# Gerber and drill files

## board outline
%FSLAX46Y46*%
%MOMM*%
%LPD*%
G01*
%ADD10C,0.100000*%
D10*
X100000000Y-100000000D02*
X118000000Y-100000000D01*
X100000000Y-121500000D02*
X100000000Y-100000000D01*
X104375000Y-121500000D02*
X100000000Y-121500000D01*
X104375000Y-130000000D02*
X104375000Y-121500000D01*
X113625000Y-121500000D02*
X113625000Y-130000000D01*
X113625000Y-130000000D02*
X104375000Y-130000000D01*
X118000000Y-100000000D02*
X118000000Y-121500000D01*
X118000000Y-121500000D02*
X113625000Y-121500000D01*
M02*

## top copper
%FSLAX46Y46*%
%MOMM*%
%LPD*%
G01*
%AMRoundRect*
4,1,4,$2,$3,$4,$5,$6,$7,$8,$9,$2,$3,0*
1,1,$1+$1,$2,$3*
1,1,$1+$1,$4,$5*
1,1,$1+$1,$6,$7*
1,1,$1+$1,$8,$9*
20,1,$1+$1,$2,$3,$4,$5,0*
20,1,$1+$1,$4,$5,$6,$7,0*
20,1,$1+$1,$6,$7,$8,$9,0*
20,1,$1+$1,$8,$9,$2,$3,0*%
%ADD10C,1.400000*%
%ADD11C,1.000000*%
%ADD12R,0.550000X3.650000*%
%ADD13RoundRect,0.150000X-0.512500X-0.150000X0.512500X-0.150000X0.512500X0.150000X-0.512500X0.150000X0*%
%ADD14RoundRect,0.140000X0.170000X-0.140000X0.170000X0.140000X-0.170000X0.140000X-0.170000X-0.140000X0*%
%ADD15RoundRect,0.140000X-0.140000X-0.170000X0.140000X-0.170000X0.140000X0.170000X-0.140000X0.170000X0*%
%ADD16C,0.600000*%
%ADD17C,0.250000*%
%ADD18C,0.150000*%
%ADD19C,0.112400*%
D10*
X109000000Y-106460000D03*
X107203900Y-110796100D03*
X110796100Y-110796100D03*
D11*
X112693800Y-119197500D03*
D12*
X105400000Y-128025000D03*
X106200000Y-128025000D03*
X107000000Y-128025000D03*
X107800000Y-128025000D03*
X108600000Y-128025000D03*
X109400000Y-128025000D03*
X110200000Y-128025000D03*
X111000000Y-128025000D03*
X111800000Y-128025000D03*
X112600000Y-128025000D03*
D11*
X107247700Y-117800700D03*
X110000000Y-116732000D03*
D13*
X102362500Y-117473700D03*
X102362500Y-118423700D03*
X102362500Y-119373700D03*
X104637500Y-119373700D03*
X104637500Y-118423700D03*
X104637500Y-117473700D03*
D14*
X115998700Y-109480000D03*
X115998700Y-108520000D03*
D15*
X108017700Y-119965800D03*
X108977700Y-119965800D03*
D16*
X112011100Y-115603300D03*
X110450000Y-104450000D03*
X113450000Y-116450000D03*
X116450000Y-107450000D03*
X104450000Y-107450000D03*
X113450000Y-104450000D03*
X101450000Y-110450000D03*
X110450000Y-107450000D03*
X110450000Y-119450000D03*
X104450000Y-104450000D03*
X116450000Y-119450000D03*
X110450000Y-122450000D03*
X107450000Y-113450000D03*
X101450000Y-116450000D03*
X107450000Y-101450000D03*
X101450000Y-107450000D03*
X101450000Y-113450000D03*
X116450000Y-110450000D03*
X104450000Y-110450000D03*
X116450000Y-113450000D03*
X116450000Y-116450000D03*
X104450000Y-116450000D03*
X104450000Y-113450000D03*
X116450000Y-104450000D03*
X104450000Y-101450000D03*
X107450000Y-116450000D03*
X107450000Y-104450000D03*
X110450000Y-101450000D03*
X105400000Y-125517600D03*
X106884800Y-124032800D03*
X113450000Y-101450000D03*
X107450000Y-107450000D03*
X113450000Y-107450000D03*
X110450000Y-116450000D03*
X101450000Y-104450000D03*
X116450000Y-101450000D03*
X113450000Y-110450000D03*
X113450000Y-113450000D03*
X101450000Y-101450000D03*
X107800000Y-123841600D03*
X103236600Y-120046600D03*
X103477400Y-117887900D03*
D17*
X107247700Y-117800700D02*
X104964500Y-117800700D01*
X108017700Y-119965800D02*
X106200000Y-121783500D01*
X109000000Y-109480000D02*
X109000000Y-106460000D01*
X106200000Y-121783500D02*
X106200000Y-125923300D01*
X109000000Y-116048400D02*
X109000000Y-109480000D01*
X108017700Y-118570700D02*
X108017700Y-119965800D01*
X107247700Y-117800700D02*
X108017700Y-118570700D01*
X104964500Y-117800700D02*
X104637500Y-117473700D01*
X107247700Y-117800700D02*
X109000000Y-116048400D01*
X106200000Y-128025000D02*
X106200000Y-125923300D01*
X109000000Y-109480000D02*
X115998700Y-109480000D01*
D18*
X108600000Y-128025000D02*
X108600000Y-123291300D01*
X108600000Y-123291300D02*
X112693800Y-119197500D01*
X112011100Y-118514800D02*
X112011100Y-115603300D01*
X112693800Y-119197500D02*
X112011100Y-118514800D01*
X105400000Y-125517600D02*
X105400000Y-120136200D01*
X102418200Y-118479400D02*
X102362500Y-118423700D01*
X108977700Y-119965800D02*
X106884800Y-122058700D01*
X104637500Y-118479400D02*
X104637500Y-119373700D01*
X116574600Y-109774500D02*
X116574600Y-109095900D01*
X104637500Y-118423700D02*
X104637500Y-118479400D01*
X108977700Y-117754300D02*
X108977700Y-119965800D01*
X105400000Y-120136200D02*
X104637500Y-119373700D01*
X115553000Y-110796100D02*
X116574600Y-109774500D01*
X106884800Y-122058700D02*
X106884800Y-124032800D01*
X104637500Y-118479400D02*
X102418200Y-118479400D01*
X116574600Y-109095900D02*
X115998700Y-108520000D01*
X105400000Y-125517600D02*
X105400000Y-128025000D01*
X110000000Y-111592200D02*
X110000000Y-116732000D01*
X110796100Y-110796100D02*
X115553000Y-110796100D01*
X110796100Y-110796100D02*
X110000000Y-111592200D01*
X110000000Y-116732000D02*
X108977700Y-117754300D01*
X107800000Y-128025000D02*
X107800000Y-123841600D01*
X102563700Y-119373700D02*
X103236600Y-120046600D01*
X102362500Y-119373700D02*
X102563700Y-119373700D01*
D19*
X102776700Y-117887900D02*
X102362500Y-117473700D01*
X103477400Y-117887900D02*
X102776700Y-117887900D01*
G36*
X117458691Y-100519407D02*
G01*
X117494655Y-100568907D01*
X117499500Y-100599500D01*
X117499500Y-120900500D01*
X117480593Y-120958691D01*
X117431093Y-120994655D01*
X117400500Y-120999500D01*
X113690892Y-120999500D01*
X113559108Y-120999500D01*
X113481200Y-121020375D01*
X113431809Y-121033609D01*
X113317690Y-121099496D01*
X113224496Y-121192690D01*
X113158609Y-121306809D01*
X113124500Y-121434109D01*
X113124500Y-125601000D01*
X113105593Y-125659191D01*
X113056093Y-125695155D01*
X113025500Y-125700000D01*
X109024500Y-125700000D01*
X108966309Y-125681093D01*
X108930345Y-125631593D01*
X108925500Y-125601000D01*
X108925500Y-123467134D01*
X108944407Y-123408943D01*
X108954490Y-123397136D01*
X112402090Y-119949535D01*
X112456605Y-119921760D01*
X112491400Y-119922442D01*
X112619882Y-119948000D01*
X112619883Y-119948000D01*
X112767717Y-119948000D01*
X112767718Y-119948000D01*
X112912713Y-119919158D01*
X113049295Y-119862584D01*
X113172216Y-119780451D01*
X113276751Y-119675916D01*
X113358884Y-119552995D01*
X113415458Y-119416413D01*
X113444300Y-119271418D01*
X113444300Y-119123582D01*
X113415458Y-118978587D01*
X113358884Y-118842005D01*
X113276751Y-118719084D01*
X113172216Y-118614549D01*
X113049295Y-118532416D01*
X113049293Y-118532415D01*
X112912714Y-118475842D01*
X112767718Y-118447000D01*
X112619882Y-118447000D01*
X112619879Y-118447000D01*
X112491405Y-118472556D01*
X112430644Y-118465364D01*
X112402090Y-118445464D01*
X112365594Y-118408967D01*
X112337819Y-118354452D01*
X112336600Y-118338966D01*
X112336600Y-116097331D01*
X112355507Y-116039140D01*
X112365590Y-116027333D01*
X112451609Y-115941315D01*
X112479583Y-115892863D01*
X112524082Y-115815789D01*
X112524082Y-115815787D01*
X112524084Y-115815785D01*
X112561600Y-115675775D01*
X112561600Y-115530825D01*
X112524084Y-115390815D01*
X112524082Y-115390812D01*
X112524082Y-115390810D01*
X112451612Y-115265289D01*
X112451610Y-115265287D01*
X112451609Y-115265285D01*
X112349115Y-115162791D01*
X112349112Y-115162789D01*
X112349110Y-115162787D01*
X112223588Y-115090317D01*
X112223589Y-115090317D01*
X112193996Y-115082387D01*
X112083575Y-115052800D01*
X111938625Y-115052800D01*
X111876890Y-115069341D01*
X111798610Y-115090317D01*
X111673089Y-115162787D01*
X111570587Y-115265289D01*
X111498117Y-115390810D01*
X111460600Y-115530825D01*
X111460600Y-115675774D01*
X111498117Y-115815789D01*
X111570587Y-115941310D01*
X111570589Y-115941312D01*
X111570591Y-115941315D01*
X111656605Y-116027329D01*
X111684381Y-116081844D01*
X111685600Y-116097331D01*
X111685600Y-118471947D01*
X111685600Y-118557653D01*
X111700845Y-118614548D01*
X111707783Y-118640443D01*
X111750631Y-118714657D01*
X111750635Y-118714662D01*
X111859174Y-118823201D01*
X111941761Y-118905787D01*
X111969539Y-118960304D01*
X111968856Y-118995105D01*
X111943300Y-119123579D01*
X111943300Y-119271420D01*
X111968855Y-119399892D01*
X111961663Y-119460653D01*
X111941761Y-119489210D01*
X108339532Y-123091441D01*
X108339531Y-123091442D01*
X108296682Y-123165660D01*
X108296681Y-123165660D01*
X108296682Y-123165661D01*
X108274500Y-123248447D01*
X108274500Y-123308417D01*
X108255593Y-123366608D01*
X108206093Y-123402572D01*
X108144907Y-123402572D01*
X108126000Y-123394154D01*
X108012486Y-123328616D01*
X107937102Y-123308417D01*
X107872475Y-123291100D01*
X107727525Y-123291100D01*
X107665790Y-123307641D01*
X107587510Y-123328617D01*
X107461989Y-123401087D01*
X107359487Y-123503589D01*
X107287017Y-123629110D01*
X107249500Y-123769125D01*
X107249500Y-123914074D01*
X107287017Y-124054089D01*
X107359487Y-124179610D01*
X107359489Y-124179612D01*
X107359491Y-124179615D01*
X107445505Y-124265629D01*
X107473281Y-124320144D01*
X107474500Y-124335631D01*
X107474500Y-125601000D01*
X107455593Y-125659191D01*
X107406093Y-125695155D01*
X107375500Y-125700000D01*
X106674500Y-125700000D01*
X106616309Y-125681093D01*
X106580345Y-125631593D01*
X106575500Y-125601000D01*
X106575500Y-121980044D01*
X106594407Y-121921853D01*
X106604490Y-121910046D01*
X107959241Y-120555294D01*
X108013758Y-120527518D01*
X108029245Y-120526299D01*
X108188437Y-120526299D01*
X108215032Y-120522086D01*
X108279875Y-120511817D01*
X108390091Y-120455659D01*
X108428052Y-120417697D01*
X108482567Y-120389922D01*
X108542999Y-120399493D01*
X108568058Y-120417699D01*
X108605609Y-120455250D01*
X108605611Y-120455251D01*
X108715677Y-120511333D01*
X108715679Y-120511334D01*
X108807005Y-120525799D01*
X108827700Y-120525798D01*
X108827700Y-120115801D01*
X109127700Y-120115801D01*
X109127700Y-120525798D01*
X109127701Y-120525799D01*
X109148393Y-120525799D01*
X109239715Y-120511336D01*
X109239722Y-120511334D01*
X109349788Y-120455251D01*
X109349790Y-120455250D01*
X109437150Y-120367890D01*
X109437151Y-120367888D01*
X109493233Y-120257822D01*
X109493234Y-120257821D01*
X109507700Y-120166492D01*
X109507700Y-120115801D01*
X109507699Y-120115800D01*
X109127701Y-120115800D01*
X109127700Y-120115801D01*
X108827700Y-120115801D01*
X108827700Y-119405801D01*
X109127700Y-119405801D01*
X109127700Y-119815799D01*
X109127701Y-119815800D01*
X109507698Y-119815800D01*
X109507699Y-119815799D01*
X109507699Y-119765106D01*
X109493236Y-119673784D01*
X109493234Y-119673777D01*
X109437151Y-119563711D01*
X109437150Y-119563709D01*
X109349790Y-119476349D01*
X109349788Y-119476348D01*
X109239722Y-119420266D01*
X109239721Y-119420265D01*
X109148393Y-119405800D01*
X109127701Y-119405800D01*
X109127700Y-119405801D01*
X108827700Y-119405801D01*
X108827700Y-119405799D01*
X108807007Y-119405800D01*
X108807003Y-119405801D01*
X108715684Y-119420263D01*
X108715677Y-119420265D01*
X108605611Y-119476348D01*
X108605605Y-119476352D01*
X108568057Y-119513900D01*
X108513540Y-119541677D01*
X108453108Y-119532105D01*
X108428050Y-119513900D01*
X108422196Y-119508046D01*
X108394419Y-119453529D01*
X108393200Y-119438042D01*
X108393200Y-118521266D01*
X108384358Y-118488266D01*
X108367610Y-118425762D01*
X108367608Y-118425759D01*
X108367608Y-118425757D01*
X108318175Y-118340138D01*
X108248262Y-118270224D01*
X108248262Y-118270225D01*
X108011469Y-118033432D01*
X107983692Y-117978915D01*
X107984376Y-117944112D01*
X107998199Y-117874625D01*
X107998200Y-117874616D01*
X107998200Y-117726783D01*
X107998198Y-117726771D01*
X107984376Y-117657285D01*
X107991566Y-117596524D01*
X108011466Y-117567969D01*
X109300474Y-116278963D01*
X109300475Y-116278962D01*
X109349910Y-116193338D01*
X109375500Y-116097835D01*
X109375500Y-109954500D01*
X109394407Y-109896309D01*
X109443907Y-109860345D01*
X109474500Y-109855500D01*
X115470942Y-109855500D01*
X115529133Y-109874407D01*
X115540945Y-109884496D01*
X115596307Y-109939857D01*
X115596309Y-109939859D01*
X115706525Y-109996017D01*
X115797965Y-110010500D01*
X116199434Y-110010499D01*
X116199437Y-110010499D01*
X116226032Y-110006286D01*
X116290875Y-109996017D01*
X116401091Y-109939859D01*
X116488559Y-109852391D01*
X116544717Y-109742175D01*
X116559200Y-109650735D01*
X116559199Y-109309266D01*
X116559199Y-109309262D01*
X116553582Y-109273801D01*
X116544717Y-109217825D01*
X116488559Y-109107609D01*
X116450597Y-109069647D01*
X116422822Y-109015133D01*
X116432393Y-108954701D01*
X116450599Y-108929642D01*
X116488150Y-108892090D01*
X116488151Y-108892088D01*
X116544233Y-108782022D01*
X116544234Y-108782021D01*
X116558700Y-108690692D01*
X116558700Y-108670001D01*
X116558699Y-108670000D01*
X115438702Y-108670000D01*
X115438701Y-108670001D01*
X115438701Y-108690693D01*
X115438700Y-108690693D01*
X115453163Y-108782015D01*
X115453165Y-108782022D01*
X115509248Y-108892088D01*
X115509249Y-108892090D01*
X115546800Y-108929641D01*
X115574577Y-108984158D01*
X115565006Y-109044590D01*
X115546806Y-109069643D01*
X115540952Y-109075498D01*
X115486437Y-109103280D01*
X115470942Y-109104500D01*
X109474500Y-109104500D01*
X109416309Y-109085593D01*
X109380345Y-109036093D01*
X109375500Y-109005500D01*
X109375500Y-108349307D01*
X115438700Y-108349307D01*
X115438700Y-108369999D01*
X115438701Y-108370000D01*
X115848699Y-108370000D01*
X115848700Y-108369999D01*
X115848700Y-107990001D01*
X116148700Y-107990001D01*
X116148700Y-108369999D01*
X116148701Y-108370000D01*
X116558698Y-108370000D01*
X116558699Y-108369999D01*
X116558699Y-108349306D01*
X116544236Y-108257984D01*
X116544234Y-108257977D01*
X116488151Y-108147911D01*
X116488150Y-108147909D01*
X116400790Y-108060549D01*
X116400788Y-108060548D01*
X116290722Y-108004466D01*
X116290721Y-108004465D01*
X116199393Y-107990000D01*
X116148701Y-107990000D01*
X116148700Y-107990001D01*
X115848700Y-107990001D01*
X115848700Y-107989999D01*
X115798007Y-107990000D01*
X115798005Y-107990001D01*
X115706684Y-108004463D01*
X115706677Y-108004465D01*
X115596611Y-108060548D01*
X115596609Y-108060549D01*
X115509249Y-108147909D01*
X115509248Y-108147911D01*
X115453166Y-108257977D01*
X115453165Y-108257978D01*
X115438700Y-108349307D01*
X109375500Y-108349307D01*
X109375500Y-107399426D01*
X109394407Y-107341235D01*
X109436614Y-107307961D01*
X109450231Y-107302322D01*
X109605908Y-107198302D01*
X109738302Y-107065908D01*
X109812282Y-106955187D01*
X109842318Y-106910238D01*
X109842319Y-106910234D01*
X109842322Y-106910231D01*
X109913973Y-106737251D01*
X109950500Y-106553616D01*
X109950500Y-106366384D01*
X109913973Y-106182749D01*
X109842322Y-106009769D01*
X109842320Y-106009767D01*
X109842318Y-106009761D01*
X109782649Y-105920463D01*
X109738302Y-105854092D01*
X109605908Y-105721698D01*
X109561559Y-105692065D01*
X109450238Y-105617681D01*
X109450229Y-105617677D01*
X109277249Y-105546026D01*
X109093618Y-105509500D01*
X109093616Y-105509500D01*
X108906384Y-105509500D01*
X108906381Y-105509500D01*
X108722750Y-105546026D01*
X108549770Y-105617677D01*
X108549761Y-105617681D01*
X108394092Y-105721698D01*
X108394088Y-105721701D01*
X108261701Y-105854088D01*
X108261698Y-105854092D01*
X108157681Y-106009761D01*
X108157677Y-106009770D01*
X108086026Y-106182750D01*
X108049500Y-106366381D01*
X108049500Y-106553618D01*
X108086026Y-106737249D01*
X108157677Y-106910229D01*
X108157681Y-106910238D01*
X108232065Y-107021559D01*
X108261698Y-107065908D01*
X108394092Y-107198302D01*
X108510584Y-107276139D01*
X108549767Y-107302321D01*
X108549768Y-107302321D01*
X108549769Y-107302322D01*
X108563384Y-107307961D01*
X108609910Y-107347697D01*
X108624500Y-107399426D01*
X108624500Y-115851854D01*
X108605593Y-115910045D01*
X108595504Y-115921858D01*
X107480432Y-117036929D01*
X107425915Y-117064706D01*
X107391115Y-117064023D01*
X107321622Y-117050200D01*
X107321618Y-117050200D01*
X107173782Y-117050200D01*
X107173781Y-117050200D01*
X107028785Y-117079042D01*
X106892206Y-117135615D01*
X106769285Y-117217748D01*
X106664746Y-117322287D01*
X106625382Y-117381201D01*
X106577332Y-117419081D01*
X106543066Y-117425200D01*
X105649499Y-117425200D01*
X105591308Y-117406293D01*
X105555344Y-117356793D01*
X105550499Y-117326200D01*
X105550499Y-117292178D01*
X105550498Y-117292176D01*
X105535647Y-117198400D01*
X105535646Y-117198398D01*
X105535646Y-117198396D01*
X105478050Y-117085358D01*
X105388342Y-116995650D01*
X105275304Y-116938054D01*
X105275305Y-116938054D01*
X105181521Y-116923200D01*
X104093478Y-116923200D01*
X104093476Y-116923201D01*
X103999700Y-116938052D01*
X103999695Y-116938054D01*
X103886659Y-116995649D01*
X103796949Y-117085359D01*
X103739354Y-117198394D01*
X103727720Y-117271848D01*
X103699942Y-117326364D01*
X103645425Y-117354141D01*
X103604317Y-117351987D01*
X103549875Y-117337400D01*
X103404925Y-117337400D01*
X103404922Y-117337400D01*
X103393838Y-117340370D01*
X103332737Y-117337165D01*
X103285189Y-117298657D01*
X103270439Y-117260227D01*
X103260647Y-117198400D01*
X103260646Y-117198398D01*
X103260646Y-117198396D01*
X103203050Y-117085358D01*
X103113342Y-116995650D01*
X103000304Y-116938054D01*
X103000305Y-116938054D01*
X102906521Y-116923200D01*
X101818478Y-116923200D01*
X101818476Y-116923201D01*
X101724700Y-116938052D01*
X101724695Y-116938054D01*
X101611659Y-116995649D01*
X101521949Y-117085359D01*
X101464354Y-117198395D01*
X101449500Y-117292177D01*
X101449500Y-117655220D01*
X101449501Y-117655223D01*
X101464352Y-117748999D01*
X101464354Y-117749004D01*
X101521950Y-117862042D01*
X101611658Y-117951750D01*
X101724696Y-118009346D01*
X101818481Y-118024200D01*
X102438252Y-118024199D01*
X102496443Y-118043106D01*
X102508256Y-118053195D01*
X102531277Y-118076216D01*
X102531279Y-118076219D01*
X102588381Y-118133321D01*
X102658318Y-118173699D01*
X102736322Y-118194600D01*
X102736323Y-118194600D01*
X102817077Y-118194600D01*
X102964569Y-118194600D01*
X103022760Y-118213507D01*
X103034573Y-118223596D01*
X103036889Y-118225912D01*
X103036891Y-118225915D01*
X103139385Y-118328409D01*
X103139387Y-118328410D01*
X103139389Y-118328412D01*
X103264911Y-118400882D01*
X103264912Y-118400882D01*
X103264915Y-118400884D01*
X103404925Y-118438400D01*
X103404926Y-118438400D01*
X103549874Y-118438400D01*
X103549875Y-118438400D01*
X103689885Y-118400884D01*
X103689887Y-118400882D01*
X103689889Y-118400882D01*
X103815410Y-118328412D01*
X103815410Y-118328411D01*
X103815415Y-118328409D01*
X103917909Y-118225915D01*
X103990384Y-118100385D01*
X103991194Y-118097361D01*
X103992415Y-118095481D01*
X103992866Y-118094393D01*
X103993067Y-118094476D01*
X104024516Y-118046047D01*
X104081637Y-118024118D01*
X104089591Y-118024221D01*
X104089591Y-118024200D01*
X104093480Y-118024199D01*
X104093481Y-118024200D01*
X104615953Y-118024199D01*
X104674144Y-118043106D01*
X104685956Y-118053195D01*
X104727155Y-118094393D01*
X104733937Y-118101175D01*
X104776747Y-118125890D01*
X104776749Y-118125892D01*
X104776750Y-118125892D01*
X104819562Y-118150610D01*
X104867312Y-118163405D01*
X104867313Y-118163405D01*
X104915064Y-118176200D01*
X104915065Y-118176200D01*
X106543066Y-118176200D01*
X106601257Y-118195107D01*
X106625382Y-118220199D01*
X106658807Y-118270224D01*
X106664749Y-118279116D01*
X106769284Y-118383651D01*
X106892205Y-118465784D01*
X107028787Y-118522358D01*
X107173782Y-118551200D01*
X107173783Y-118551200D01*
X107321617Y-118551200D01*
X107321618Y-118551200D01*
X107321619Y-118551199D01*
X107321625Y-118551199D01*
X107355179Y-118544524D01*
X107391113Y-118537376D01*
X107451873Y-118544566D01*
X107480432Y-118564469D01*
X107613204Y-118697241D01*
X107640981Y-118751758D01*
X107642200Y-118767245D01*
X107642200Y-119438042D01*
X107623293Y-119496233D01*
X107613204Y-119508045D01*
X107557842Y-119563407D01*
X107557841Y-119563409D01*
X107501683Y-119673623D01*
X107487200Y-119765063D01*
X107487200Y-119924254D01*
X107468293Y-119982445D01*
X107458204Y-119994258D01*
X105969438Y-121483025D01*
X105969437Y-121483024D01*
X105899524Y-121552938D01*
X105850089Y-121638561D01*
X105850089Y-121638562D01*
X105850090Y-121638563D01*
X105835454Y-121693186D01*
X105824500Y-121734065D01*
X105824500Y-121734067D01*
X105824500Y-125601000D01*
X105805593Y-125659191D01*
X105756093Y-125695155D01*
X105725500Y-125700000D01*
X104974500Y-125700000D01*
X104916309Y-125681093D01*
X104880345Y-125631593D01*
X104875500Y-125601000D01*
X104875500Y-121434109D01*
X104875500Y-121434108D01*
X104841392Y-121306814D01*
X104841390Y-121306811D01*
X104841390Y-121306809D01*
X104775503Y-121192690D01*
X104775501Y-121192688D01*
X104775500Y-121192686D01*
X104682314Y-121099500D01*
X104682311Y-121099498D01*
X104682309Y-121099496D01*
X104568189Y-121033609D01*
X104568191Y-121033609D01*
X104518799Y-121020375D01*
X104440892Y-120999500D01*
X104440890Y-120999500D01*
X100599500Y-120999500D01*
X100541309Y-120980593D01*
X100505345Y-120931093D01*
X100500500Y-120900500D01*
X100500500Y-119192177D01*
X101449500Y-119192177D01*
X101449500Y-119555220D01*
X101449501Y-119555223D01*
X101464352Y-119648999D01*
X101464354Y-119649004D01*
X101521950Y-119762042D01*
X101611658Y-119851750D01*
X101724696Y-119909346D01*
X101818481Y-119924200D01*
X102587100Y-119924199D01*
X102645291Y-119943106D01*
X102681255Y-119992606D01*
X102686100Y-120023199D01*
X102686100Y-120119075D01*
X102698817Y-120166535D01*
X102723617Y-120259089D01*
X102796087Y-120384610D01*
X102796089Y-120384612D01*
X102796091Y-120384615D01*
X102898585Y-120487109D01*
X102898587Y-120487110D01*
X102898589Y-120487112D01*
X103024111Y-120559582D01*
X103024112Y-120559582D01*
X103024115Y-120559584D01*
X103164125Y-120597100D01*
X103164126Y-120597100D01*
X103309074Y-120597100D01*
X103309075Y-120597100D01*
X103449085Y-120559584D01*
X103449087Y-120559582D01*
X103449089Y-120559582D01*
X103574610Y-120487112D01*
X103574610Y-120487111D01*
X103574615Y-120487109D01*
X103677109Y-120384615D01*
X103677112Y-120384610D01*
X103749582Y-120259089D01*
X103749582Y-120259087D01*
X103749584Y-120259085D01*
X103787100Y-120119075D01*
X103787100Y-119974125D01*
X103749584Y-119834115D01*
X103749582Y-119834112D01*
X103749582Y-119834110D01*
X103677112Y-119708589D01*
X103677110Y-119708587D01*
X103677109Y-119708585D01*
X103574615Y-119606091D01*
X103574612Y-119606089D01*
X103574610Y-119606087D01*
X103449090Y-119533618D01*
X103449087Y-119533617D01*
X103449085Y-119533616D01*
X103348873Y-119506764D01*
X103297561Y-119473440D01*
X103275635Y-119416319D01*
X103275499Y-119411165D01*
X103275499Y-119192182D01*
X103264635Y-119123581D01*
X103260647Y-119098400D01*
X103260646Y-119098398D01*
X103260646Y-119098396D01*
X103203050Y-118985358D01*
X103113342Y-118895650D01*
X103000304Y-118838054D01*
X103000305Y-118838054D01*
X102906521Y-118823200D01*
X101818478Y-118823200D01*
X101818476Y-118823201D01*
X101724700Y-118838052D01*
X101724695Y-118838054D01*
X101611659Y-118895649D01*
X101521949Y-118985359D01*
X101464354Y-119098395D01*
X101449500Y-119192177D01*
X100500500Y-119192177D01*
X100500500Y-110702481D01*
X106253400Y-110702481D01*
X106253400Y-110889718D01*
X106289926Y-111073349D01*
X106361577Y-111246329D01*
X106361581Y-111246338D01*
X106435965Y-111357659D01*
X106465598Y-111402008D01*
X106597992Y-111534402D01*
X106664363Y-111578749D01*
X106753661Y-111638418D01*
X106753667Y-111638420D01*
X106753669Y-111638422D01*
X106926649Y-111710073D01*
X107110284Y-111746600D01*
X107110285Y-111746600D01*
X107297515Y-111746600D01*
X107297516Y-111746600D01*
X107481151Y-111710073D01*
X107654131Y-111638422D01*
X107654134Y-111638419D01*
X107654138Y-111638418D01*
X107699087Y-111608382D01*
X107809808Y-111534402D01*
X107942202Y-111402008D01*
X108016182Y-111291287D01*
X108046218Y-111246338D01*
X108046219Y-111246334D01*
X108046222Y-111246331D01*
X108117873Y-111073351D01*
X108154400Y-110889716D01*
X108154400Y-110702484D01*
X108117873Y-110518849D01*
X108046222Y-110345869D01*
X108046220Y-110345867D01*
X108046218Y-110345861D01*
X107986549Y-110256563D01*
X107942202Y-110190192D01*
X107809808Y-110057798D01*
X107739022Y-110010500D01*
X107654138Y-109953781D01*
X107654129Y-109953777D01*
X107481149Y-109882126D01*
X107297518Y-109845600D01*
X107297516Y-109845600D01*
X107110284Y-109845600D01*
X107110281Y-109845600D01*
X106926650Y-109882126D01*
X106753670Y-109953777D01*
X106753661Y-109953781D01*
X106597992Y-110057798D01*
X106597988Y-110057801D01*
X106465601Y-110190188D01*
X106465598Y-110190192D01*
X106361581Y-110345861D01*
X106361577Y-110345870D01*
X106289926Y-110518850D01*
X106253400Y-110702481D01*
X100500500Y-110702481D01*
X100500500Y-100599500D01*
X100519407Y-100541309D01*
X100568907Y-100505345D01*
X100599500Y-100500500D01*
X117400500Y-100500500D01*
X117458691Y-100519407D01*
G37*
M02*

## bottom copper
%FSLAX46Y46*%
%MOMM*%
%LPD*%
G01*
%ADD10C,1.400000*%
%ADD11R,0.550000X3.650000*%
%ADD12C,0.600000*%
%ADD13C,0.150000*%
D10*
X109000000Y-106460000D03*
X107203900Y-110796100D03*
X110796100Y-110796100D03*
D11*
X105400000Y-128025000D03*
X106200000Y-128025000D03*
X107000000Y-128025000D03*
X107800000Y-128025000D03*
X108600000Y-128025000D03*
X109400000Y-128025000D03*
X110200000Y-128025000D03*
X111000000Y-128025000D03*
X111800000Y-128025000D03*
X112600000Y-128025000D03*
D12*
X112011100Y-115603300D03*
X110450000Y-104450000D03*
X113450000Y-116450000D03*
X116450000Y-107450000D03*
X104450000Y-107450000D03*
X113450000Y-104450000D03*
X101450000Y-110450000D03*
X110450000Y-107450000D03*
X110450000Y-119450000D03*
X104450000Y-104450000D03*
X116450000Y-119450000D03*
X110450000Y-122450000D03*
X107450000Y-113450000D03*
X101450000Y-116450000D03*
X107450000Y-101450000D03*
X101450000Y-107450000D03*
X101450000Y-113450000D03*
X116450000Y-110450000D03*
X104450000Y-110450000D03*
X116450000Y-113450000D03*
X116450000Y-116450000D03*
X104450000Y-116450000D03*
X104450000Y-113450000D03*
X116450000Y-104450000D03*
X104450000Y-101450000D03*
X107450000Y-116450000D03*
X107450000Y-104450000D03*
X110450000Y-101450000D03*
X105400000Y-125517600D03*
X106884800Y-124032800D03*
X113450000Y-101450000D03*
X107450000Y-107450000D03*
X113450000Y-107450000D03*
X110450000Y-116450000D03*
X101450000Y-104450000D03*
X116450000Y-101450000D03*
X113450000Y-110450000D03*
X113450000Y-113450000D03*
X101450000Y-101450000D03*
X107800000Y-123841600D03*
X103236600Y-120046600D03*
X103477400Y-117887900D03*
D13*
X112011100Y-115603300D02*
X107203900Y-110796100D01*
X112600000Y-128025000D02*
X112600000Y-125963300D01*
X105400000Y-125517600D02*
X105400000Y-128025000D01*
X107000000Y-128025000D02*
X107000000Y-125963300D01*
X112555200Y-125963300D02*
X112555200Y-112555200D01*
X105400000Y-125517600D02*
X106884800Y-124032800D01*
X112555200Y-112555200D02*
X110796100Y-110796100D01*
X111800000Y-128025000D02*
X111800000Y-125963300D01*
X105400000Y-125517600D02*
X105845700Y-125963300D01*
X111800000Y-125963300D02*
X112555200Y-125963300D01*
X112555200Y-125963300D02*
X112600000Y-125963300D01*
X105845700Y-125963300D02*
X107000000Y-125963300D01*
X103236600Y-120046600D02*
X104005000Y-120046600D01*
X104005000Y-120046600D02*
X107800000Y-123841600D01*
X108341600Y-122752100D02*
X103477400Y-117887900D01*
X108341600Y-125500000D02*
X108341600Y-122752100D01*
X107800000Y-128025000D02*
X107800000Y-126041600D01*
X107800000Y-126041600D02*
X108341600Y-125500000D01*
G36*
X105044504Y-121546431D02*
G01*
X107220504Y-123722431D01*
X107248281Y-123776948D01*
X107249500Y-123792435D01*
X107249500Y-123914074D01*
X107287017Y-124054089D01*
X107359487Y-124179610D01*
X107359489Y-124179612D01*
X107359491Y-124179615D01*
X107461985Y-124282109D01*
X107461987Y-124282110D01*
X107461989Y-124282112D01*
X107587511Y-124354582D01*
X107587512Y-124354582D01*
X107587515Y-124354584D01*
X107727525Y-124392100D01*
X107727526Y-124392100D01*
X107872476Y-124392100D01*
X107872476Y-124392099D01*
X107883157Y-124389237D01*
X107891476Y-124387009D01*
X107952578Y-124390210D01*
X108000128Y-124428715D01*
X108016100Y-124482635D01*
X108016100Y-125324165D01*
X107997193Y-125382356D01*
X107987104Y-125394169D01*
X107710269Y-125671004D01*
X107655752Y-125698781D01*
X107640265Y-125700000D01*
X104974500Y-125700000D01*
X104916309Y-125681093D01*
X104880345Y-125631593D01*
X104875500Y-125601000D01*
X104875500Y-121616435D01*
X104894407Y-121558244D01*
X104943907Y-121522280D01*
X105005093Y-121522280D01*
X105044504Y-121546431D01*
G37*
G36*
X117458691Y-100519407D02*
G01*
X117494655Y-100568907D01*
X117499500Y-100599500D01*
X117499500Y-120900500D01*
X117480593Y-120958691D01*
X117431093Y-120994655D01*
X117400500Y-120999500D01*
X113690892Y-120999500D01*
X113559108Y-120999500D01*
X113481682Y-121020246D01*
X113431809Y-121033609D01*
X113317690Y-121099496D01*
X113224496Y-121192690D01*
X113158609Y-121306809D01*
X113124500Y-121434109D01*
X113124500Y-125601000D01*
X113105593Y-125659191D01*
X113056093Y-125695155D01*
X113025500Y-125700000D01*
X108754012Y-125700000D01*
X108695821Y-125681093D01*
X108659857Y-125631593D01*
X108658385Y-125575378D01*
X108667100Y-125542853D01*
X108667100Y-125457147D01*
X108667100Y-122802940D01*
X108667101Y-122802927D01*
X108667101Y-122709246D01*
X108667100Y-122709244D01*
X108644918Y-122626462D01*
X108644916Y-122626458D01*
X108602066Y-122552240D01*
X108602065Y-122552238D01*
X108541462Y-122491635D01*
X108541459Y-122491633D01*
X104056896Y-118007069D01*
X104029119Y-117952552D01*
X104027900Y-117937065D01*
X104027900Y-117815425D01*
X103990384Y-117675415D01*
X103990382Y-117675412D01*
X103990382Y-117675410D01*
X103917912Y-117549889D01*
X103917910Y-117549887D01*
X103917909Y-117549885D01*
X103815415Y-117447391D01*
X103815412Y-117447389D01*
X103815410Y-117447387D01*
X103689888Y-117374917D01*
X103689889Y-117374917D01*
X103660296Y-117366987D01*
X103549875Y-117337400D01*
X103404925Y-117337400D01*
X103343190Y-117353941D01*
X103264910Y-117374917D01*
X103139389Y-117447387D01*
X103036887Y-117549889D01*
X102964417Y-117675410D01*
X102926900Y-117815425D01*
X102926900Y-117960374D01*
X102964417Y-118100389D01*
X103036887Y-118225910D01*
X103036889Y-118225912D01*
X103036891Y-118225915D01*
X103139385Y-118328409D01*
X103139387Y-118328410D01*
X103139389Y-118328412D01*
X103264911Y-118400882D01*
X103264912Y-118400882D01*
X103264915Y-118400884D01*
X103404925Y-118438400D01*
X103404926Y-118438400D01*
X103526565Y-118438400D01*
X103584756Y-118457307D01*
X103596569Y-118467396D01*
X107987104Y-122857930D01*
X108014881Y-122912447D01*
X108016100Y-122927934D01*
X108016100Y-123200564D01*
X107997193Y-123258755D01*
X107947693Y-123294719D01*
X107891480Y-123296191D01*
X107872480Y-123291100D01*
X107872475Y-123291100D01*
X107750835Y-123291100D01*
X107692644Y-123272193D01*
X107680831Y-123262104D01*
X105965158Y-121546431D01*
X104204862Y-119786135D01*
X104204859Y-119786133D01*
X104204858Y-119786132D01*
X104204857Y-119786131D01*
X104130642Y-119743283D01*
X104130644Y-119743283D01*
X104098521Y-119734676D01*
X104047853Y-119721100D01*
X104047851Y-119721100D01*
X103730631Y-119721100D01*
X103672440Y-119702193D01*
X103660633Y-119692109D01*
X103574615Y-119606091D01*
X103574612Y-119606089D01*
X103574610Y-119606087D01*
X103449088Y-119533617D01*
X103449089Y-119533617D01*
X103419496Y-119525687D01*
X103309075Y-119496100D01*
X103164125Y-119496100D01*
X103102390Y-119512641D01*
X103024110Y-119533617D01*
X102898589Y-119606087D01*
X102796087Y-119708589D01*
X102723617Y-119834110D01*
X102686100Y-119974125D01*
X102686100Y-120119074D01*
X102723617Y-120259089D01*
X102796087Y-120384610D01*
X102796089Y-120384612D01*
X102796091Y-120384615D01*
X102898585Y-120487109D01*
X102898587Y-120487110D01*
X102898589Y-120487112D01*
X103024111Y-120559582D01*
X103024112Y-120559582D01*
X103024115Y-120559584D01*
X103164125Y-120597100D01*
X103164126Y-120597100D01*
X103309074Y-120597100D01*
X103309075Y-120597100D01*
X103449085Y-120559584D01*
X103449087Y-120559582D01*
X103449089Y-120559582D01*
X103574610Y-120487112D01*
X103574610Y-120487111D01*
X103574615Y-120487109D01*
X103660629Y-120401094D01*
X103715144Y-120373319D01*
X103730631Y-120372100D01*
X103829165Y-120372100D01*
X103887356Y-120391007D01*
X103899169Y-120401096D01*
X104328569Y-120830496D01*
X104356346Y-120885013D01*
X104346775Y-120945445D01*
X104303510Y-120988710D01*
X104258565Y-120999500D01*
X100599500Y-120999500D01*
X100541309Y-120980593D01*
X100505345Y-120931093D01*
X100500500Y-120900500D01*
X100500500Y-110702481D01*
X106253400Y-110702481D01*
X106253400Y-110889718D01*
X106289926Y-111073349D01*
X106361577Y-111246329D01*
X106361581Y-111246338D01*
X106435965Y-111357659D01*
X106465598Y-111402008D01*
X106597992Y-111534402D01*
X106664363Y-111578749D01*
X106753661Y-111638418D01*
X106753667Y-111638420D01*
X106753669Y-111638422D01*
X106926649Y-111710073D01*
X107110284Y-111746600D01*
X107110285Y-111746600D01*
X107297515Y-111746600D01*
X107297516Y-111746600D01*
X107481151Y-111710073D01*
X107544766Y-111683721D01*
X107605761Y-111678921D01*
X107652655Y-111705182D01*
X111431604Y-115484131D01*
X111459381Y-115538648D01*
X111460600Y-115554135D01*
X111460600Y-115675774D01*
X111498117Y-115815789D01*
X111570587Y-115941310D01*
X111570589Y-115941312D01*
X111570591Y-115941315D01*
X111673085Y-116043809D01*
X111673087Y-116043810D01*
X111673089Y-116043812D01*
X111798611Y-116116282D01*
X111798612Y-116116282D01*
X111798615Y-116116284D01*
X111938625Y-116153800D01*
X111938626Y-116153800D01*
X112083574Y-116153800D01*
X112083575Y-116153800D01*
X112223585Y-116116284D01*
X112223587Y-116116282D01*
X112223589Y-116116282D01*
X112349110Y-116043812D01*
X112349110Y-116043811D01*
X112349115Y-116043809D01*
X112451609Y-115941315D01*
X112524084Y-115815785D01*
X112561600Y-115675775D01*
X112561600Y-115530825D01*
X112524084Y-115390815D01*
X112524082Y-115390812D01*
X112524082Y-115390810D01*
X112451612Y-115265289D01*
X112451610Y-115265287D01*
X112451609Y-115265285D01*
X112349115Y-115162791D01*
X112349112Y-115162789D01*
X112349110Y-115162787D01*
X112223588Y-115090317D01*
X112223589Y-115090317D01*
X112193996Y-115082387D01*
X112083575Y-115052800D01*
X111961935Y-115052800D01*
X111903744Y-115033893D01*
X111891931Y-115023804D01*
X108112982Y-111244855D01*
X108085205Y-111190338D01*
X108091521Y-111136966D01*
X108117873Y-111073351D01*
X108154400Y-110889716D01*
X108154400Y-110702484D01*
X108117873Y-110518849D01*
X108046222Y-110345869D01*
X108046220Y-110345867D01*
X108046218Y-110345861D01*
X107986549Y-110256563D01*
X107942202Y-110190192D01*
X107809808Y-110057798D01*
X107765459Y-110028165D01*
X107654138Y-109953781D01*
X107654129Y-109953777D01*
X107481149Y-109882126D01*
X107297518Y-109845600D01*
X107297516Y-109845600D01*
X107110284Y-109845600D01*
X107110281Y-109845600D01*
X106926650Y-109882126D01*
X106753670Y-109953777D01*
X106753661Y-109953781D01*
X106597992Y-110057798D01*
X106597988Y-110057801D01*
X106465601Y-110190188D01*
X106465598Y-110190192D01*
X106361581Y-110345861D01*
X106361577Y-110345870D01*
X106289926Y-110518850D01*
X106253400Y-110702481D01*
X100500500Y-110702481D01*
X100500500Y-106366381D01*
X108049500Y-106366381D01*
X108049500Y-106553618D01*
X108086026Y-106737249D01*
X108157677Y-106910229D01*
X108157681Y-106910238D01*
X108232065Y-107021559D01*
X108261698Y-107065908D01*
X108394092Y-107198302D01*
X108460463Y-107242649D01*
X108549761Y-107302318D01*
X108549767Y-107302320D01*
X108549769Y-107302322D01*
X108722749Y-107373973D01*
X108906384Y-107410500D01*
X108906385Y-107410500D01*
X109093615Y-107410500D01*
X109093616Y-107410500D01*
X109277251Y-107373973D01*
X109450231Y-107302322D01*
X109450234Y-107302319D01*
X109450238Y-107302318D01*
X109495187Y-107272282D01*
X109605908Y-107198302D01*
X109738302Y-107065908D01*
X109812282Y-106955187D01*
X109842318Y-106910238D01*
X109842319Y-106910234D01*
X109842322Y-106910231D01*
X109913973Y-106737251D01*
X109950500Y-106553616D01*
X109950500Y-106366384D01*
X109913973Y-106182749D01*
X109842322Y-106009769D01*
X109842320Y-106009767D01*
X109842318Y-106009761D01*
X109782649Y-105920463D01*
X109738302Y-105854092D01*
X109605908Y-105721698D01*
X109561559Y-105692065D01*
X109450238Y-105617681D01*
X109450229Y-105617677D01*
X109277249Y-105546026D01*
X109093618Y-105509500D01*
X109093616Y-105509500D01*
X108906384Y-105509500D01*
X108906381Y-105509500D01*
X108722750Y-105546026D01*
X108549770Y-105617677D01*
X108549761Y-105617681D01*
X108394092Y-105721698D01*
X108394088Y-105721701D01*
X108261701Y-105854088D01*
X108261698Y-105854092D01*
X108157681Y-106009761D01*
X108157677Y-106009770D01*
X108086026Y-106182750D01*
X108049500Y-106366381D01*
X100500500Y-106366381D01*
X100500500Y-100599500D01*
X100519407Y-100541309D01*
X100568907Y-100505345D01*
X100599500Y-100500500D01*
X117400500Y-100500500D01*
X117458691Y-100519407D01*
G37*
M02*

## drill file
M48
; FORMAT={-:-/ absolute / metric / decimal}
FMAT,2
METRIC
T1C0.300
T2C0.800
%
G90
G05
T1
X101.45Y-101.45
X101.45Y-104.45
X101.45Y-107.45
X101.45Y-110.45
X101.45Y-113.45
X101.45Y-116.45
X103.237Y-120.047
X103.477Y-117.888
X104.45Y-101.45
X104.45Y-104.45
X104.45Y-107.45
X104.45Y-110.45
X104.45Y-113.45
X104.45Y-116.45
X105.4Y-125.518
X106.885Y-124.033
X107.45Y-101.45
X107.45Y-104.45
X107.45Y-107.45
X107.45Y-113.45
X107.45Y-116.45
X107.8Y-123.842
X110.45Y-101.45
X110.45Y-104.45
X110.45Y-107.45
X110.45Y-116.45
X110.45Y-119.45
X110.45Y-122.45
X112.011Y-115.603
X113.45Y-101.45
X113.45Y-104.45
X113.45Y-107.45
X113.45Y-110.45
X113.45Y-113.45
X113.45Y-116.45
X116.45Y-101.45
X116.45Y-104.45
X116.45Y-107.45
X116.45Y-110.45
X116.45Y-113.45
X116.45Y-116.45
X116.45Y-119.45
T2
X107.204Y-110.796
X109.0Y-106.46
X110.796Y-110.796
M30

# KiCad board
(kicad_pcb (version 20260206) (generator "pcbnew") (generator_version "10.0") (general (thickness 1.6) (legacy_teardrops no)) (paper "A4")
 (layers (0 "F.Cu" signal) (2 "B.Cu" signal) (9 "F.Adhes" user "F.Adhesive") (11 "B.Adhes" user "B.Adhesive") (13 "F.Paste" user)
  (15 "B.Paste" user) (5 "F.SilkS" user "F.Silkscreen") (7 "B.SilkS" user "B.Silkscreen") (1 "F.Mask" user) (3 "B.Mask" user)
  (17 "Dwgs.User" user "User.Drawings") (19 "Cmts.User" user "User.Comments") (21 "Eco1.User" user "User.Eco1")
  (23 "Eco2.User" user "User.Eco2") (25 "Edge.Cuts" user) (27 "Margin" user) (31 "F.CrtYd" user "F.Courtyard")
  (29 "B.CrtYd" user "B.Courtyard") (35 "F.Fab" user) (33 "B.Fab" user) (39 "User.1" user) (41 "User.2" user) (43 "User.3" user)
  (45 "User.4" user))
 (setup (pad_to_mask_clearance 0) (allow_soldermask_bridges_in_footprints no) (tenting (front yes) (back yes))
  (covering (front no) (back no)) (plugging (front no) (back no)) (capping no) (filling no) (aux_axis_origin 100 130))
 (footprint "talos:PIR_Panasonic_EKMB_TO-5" (layer "F.Cu") (at 109 109)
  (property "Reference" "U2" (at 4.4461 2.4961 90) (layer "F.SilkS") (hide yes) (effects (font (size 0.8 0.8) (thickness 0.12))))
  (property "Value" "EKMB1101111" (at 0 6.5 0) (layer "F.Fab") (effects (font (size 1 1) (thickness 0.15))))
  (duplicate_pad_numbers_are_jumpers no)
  (pad "1" thru_hole circle (at 0 -2.54) (size 1.4 1.4) (drill 0.8) (layers "*.Cu" "*.Mask") (remove_unused_layers no) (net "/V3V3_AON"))
  (pad "2" thru_hole circle (at -1.7961 1.7961) (size 1.4 1.4) (drill 0.8) (layers "*.Cu" "*.Mask") (remove_unused_layers no) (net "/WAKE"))
  (pad "3" thru_hole circle (at 1.7961 1.7961) (size 1.4 1.4) (drill 0.8) (layers "*.Cu" "*.Mask") (remove_unused_layers no) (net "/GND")))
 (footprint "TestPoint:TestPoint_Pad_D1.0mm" (layer "F.Cu") (at 112.6938 119.1975)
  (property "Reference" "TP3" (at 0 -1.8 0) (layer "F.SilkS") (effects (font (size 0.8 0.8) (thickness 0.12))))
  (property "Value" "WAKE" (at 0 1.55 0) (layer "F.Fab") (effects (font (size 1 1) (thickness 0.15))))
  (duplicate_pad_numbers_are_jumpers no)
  (pad "1" smd circle (at 0 0) (size 1 1) (layers "F.Cu" "F.Mask") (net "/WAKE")))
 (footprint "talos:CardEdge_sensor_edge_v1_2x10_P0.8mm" (layer "F.Cu") (at 109 128.35)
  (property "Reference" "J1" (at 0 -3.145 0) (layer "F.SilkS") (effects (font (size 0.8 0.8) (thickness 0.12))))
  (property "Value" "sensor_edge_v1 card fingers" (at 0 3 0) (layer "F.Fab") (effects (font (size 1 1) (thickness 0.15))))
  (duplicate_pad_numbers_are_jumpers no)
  (pad "1" smd rect (at -3.6 -0.325) (size 0.55 3.65) (layers "F.Cu" "F.Mask") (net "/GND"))
  (pad "2" smd rect (at -3.6 -0.325) (size 0.55 3.65) (layers "B.Cu" "B.Mask") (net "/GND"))
  (pad "3" smd rect (at -2.8 -0.325) (size 0.55 3.65) (layers "F.Cu" "F.Mask") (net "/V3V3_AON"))
  (pad "4" smd rect (at -2.8 -0.325) (size 0.55 3.65) (layers "B.Cu" "B.Mask") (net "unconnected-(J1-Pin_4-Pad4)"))
  (pad "5" smd rect (at -2 -0.325) (size 0.55 3.65) (layers "F.Cu" "F.Mask") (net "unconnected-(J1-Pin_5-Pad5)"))
  (pad "6" smd rect (at -2 -0.325) (size 0.55 3.65) (layers "B.Cu" "B.Mask") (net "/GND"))
  (pad "7" smd rect (at -1.2 -0.325) (size 0.55 3.65) (layers "F.Cu" "F.Mask") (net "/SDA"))
  (pad "8" smd rect (at -1.2 -0.325) (size 0.55 3.65) (layers "B.Cu" "B.Mask") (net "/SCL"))
  (pad "9" smd rect (at -0.4 -0.325) (size 0.55 3.65) (layers "F.Cu" "F.Mask") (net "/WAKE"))
  (pad "10" smd rect (at -0.4 -0.325) (size 0.55 3.65) (layers "B.Cu" "B.Mask") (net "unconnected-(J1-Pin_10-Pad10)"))
  (pad "11" smd rect (at 0.4 -0.325) (size 0.55 3.65) (layers "F.Cu" "F.Mask") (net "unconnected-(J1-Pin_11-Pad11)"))
  (pad "12" smd rect (at 0.4 -0.325) (size 0.55 3.65) (layers "B.Cu" "B.Mask") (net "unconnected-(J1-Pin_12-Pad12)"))
  (pad "13" smd rect (at 1.2 -0.325) (size 0.55 3.65) (layers "F.Cu" "F.Mask") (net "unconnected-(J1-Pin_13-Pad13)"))
  (pad "14" smd rect (at 1.2 -0.325) (size 0.55 3.65) (layers "B.Cu" "B.Mask") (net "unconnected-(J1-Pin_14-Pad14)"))
  (pad "15" smd rect (at 2 -0.325) (size 0.55 3.65) (layers "F.Cu" "F.Mask") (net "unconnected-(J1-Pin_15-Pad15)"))
  (pad "16" smd rect (at 2 -0.325) (size 0.55 3.65) (layers "B.Cu" "B.Mask") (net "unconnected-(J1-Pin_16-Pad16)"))
  (pad "17" smd rect (at 2.8 -0.325) (size 0.55 3.65) (layers "F.Cu" "F.Mask") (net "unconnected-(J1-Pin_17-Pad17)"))
  (pad "18" smd rect (at 2.8 -0.325) (size 0.55 3.65) (layers "B.Cu" "B.Mask") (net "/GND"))
  (pad "19" smd rect (at 3.6 -0.325) (size 0.55 3.65) (layers "F.Cu" "F.Mask") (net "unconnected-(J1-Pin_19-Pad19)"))
  (pad "20" smd rect (at 3.6 -0.325) (size 0.55 3.65) (layers "B.Cu" "B.Mask") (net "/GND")))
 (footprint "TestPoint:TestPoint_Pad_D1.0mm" (layer "F.Cu") (at 107.2477 117.8007)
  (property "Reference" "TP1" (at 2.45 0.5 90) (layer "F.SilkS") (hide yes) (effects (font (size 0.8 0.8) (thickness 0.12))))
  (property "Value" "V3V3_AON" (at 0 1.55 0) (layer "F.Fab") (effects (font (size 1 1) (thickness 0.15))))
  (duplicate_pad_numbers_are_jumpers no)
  (pad "1" smd circle (at 0 0) (size 1 1) (layers "F.Cu" "F.Mask") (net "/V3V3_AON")))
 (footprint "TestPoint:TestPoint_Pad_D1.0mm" (layer "F.Cu") (at 110 116.732)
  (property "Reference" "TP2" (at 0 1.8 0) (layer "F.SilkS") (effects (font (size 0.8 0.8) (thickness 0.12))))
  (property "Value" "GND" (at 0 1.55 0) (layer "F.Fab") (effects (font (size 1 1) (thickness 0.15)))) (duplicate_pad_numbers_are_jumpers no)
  (pad "1" smd circle (at 0 0) (size 1 1) (layers "F.Cu" "F.Mask") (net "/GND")))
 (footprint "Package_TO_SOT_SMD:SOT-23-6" (layer "F.Cu") (at 103.5 118.4237)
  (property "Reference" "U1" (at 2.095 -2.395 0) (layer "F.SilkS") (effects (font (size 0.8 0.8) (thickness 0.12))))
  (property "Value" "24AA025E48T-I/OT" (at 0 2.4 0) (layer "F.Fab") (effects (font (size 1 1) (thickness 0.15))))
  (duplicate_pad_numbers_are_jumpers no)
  (pad "1" smd roundrect (at -1.1375 -0.95) (size 1.325 0.6) (layers "F.Cu" "F.Mask" "F.Paste") (roundrect_rratio 0.25) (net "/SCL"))
  (pad "2" smd roundrect (at -1.1375 0) (size 1.325 0.6) (layers "F.Cu" "F.Mask" "F.Paste") (roundrect_rratio 0.25) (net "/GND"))
  (pad "3" smd roundrect (at -1.1375 0.95) (size 1.325 0.6) (layers "F.Cu" "F.Mask" "F.Paste") (roundrect_rratio 0.25) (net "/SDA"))
  (pad "4" smd roundrect (at 1.1375 0.95) (size 1.325 0.6) (layers "F.Cu" "F.Mask" "F.Paste") (roundrect_rratio 0.25) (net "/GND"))
  (pad "5" smd roundrect (at 1.1375 0) (size 1.325 0.6) (layers "F.Cu" "F.Mask" "F.Paste") (roundrect_rratio 0.25) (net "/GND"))
  (pad "6" smd roundrect (at 1.1375 -0.95) (size 1.325 0.6) (layers "F.Cu" "F.Mask" "F.Paste") (roundrect_rratio 0.25) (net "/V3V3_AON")))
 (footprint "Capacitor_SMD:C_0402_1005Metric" (layer "F.Cu") (at 115.9987 109 90)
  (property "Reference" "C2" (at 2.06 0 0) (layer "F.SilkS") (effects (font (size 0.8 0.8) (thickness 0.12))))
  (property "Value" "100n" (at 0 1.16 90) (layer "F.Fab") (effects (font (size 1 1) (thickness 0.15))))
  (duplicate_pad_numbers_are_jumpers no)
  (pad "1" smd roundrect (at -0.48 0 90) (size 0.56 0.62) (layers "F.Cu" "F.Mask" "F.Paste") (roundrect_rratio 0.25) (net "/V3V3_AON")
   (zone_connect 1))
  (pad "2" smd roundrect (at 0.48 0 90) (size 0.56 0.62) (layers "F.Cu" "F.Mask" "F.Paste") (roundrect_rratio 0.25) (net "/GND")
   (zone_connect 1)))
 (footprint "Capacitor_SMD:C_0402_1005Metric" (layer "F.Cu") (at 108.4977 119.9658)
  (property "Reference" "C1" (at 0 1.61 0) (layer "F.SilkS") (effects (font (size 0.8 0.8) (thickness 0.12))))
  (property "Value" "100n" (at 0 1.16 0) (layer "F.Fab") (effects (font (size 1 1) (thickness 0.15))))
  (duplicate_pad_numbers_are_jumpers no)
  (pad "1" smd roundrect (at -0.48 0) (size 0.56 0.62) (layers "F.Cu" "F.Mask" "F.Paste") (roundrect_rratio 0.25) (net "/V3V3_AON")
   (zone_connect 1))
  (pad "2" smd roundrect (at 0.48 0) (size 0.56 0.62) (layers "F.Cu" "F.Mask" "F.Paste") (roundrect_rratio 0.25) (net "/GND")
   (zone_connect 1)))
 (gr_line (start 100 100) (end 118 100) (stroke (width 0.1) (type default)) (layer "Edge.Cuts"))
 (gr_line (start 100 121.5) (end 100 100) (stroke (width 0.1) (type default)) (layer "Edge.Cuts"))
 (gr_line (start 104.375 121.5) (end 100 121.5) (stroke (width 0.1) (type default)) (layer "Edge.Cuts"))
 (gr_line (start 104.375 130) (end 104.375 121.5) (stroke (width 0.1) (type default)) (layer "Edge.Cuts"))
 (gr_line (start 113.625 121.5) (end 113.625 130) (stroke (width 0.1) (type default)) (layer "Edge.Cuts"))
 (gr_line (start 113.625 130) (end 104.375 130) (stroke (width 0.1) (type default)) (layer "Edge.Cuts"))
 (gr_line (start 118 100) (end 118 121.5) (stroke (width 0.1) (type default)) (layer "Edge.Cuts"))
 (gr_line (start 118 121.5) (end 113.625 121.5) (stroke (width 0.1) (type default)) (layer "Edge.Cuts"))
 (segment (start 107.2477 117.8007) (end 104.9645 117.8007) (width 0.25) (layer "F.Cu") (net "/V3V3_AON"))
 (segment (start 108.0177 119.9658) (end 106.2 121.7835) (width 0.25) (layer "F.Cu") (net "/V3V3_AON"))
 (segment (start 109 109.48) (end 109 106.46) (width 0.25) (layer "F.Cu") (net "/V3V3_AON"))
 (segment (start 106.2 121.7835) (end 106.2 125.9233) (width 0.25) (layer "F.Cu") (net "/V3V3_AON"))
 (segment (start 109 116.0484) (end 109 109.48) (width 0.25) (layer "F.Cu") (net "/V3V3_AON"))
 (segment (start 108.0177 118.5707) (end 108.0177 119.9658) (width 0.25) (layer "F.Cu") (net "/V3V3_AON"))
 (segment (start 107.2477 117.8007) (end 108.0177 118.5707) (width 0.25) (layer "F.Cu") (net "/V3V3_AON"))
 (segment (start 104.9645 117.8007) (end 104.6375 117.4737) (width 0.25) (layer "F.Cu") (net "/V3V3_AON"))
 (segment (start 107.2477 117.8007) (end 109 116.0484) (width 0.25) (layer "F.Cu") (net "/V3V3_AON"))
 (segment (start 106.2 128.025) (end 106.2 125.9233) (width 0.25) (layer "F.Cu") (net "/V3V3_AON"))
 (segment (start 109 109.48) (end 115.9987 109.48) (width 0.25) (layer "F.Cu") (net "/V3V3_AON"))
 (segment (start 108.6 128.025) (end 108.6 123.2913) (width 0.15) (layer "F.Cu") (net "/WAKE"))
 (segment (start 108.6 123.2913) (end 112.6938 119.1975) (width 0.15) (layer "F.Cu") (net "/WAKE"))
 (segment (start 112.0111 118.5148) (end 112.0111 115.6033) (width 0.15) (layer "F.Cu") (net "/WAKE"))
 (segment (start 112.6938 119.1975) (end 112.0111 118.5148) (width 0.15) (layer "F.Cu") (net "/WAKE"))
 (via (at 112.0111 115.6033) (size 0.6) (drill 0.3) (layers "F.Cu" "B.Cu") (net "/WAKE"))
 (segment (start 112.0111 115.6033) (end 107.2039 110.7961) (width 0.15) (layer "B.Cu") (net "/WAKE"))
 (segment (start 105.4 125.5176) (end 105.4 120.1362) (width 0.15) (layer "F.Cu") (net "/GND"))
 (segment (start 102.4182 118.4794) (end 102.3625 118.4237) (width 0.15) (layer "F.Cu") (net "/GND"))
 (segment (start 108.9777 119.9658) (end 106.8848 122.0587) (width 0.15) (layer "F.Cu") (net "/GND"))
 (segment (start 104.6375 118.4794) (end 104.6375 119.3737) (width 0.15) (layer "F.Cu") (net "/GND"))
 (segment (start 116.5746 109.7745) (end 116.5746 109.0959) (width 0.15) (layer "F.Cu") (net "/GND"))
 (segment (start 104.6375 118.4237) (end 104.6375 118.4794) (width 0.15) (layer "F.Cu") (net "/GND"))
 (segment (start 108.9777 117.7543) (end 108.9777 119.9658) (width 0.15) (layer "F.Cu") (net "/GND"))
 (segment (start 105.4 120.1362) (end 104.6375 119.3737) (width 0.15) (layer "F.Cu") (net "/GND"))
 (segment (start 115.553 110.7961) (end 116.5746 109.7745) (width 0.15) (layer "F.Cu") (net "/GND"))
 (segment (start 106.8848 122.0587) (end 106.8848 124.0328) (width 0.15) (layer "F.Cu") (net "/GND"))
 (segment (start 104.6375 118.4794) (end 102.4182 118.4794) (width 0.15) (layer "F.Cu") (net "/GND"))
 (segment (start 116.5746 109.0959) (end 115.9987 108.52) (width 0.15) (layer "F.Cu") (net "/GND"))
 (segment (start 105.4 125.5176) (end 105.4 128.025) (width 0.15) (layer "F.Cu") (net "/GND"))
 (segment (start 110 111.5922) (end 110 116.732) (width 0.15) (layer "F.Cu") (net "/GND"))
 (segment (start 110.7961 110.7961) (end 115.553 110.7961) (width 0.15) (layer "F.Cu") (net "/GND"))
 (segment (start 110.7961 110.7961) (end 110 111.5922) (width 0.15) (layer "F.Cu") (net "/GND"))
 (segment (start 110 116.732) (end 108.9777 117.7543) (width 0.15) (layer "F.Cu") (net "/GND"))
 (via (at 110.45 104.45) (size 0.6) (drill 0.3) (layers "F.Cu" "B.Cu") (locked yes) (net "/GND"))
 (via (at 113.45 116.45) (size 0.6) (drill 0.3) (layers "F.Cu" "B.Cu") (locked yes) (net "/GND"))
 (via (at 116.45 107.45) (size 0.6) (drill 0.3) (layers "F.Cu" "B.Cu") (locked yes) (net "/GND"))
 (via (at 104.45 107.45) (size 0.6) (drill 0.3) (layers "F.Cu" "B.Cu") (locked yes) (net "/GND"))
 (via (at 113.45 104.45) (size 0.6) (drill 0.3) (layers "F.Cu" "B.Cu") (locked yes) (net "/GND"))
 (via (at 101.45 110.45) (size 0.6) (drill 0.3) (layers "F.Cu" "B.Cu") (locked yes) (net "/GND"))
 (via (at 110.45 107.45) (size 0.6) (drill 0.3) (layers "F.Cu" "B.Cu") (locked yes) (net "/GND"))
 (via (at 110.45 119.45) (size 0.6) (drill 0.3) (layers "F.Cu" "B.Cu") (locked yes) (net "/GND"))
 (via (at 104.45 104.45) (size 0.6) (drill 0.3) (layers "F.Cu" "B.Cu") (locked yes) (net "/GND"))
 (via (at 116.45 119.45) (size 0.6) (drill 0.3) (layers "F.Cu" "B.Cu") (locked yes) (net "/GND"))
 (via (at 110.45 122.45) (size 0.6) (drill 0.3) (layers "F.Cu" "B.Cu") (locked yes) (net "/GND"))
 (via (at 107.45 113.45) (size 0.6) (drill 0.3) (layers "F.Cu" "B.Cu") (locked yes) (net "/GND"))
 (via (at 101.45 116.45) (size 0.6) (drill 0.3) (layers "F.Cu" "B.Cu") (locked yes) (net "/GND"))
 (via (at 107.45 101.45) (size 0.6) (drill 0.3) (layers "F.Cu" "B.Cu") (locked yes) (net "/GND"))
 (via (at 101.45 107.45) (size 0.6) (drill 0.3) (layers "F.Cu" "B.Cu") (locked yes) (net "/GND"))
 (via (at 101.45 113.45) (size 0.6) (drill 0.3) (layers "F.Cu" "B.Cu") (locked yes) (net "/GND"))
 (via (at 116.45 110.45) (size 0.6) (drill 0.3) (layers "F.Cu" "B.Cu") (locked yes) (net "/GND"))
 (via (at 104.45 110.45) (size 0.6) (drill 0.3) (layers "F.Cu" "B.Cu") (locked yes) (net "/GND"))
 (via (at 116.45 113.45) (size 0.6) (drill 0.3) (layers "F.Cu" "B.Cu") (locked yes) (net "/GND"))
 (via (at 116.45 116.45) (size 0.6) (drill 0.3) (layers "F.Cu" "B.Cu") (locked yes) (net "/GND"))
 (via (at 104.45 116.45) (size 0.6) (drill 0.3) (layers "F.Cu" "B.Cu") (locked yes) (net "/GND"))
 (via (at 104.45 113.45) (size 0.6) (drill 0.3) (layers "F.Cu" "B.Cu") (locked yes) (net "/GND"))
 (via (at 116.45 104.45) (size 0.6) (drill 0.3) (layers "F.Cu" "B.Cu") (locked yes) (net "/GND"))
 (via (at 104.45 101.45) (size 0.6) (drill 0.3) (layers "F.Cu" "B.Cu") (locked yes) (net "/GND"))
 (via (at 107.45 116.45) (size 0.6) (drill 0.3) (layers "F.Cu" "B.Cu") (locked yes) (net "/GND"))
 (via (at 107.45 104.45) (size 0.6) (drill 0.3) (layers "F.Cu" "B.Cu") (locked yes) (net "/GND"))
 (via (at 110.45 101.45) (size 0.6) (drill 0.3) (layers "F.Cu" "B.Cu") (locked yes) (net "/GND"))
 (via (at 105.4 125.5176) (size 0.6) (drill 0.3) (layers "F.Cu" "B.Cu") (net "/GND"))
 (via (at 106.8848 124.0328) (size 0.6) (drill 0.3) (layers "F.Cu" "B.Cu") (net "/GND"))
 (via (at 113.45 101.45) (size 0.6) (drill 0.3) (layers "F.Cu" "B.Cu") (locked yes) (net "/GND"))
 (via (at 107.45 107.45) (size 0.6) (drill 0.3) (layers "F.Cu" "B.Cu") (locked yes) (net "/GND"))
 (via (at 113.45 107.45) (size 0.6) (drill 0.3) (layers "F.Cu" "B.Cu") (locked yes) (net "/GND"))
 (via (at 110.45 116.45) (size 0.6) (drill 0.3) (layers "F.Cu" "B.Cu") (locked yes) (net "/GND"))
 (via (at 101.45 104.45) (size 0.6) (drill 0.3) (layers "F.Cu" "B.Cu") (locked yes) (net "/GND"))
 (via (at 116.45 101.45) (size 0.6) (drill 0.3) (layers "F.Cu" "B.Cu") (locked yes) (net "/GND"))
 (via (at 113.45 110.45) (size 0.6) (drill 0.3) (layers "F.Cu" "B.Cu") (locked yes) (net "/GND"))
 (via (at 113.45 113.45) (size 0.6) (drill 0.3) (layers "F.Cu" "B.Cu") (locked yes) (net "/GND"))
 (via (at 101.45 101.45) (size 0.6) (drill 0.3) (layers "F.Cu" "B.Cu") (locked yes) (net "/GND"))
 (segment (start 112.6 128.025) (end 112.6 125.9633) (width 0.15) (layer "B.Cu") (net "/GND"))
 (segment (start 105.4 125.5176) (end 105.4 128.025) (width 0.15) (layer "B.Cu") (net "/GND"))
 (segment (start 107 128.025) (end 107 125.9633) (width 0.15) (layer "B.Cu") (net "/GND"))
 (segment (start 112.5552 125.9633) (end 112.5552 112.5552) (width 0.15) (layer "B.Cu") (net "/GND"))
 (segment (start 105.4 125.5176) (end 106.8848 124.0328) (width 0.15) (layer "B.Cu") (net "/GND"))
 (segment (start 112.5552 112.5552) (end 110.7961 110.7961) (width 0.15) (layer "B.Cu") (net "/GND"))
 (segment (start 111.8 128.025) (end 111.8 125.9633) (width 0.15) (layer "B.Cu") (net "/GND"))
 (segment (start 105.4 125.5176) (end 105.8457 125.9633) (width 0.15) (layer "B.Cu") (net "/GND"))
 (segment (start 111.8 125.9633) (end 112.5552 125.9633) (width 0.15) (layer "B.Cu") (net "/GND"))
 (segment (start 112.5552 125.9633) (end 112.6 125.9633) (width 0.15) (layer "B.Cu") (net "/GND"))
 (segment (start 105.8457 125.9633) (end 107 125.9633) (width 0.15) (layer "B.Cu") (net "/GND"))
 (segment (start 107.8 128.025) (end 107.8 123.8416) (width 0.15) (layer "F.Cu") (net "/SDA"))
 (segment (start 102.5637 119.3737) (end 103.2366 120.0466) (width 0.15) (layer "F.Cu") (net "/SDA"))
 (segment (start 102.3625 119.3737) (end 102.5637 119.3737) (width 0.15) (layer "F.Cu") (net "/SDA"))
 (via (at 107.8 123.8416) (size 0.6) (drill 0.3) (layers "F.Cu" "B.Cu") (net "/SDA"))
 (via (at 103.2366 120.0466) (size 0.6) (drill 0.3) (layers "F.Cu" "B.Cu") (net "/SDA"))
 (segment (start 103.2366 120.0466) (end 104.005 120.0466) (width 0.15) (layer "B.Cu") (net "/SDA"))
 (segment (start 104.005 120.0466) (end 107.8 123.8416) (width 0.15) (layer "B.Cu") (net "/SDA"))
 (segment (start 102.7767 117.8879) (end 102.3625 117.4737) (width 0.1124) (layer "F.Cu") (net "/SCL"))
 (segment (start 103.4774 117.8879) (end 102.7767 117.8879) (width 0.1124) (layer "F.Cu") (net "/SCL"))
 (via (at 103.4774 117.8879) (size 0.6) (drill 0.3) (layers "F.Cu" "B.Cu") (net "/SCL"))
 (segment (start 108.3416 122.7521) (end 103.4774 117.8879) (width 0.15) (layer "B.Cu") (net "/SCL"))
 (segment (start 108.3416 125.5) (end 108.3416 122.7521) (width 0.15) (layer "B.Cu") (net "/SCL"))
 (segment (start 107.8 128.025) (end 107.8 126.0416) (width 0.15) (layer "B.Cu") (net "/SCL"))
 (segment (start 107.8 126.0416) (end 108.3416 125.5) (width 0.15) (layer "B.Cu") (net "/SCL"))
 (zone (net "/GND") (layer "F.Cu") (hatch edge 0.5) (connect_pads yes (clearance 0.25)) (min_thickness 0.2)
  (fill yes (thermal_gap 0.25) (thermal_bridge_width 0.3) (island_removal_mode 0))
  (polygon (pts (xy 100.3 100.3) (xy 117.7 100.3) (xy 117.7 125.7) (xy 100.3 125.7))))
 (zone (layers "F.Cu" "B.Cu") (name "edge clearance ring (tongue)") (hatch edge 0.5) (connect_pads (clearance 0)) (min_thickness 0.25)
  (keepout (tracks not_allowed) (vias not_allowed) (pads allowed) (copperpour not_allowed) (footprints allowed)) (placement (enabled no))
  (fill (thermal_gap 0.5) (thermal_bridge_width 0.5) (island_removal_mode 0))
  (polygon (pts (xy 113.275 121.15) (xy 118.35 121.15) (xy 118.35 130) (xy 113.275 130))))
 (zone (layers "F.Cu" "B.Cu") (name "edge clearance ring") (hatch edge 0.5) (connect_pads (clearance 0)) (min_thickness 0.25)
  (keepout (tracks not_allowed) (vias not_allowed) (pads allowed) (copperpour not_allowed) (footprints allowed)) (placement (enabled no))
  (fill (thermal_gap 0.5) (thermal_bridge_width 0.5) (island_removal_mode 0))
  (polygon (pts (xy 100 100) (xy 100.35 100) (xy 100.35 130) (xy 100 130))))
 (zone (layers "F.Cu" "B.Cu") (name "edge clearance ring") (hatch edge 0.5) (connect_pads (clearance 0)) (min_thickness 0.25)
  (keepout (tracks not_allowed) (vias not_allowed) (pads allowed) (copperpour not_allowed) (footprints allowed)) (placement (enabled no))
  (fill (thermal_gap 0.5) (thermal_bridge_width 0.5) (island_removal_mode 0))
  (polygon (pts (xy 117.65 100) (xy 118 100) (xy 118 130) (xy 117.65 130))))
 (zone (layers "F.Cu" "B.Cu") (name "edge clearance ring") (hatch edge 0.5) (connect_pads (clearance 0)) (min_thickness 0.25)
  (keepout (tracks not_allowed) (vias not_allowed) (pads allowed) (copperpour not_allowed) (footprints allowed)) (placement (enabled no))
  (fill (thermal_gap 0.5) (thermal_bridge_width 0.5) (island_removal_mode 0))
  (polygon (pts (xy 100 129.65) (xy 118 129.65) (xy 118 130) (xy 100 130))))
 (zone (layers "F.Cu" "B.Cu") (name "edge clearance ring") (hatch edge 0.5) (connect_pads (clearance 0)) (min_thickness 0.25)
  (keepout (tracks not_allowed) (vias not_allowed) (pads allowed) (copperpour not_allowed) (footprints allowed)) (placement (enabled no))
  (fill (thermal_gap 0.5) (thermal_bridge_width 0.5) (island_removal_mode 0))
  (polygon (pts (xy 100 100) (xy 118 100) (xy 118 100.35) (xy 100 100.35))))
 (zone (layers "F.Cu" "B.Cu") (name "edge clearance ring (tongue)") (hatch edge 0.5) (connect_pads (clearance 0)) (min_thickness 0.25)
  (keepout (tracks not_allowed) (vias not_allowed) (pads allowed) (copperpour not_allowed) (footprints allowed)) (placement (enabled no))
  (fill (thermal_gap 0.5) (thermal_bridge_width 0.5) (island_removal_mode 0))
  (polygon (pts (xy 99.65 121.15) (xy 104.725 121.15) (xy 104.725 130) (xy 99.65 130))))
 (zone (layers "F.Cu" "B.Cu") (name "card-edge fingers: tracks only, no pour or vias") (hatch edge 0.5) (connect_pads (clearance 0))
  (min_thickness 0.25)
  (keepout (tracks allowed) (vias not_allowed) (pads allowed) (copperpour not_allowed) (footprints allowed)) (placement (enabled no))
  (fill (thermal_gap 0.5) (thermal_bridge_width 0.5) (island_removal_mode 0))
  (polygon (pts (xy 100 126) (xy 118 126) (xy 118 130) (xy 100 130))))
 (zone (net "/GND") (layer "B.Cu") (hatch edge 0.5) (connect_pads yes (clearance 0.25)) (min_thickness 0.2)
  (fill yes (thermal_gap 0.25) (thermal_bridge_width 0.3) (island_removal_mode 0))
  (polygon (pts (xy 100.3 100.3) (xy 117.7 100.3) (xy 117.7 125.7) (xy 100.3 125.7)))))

